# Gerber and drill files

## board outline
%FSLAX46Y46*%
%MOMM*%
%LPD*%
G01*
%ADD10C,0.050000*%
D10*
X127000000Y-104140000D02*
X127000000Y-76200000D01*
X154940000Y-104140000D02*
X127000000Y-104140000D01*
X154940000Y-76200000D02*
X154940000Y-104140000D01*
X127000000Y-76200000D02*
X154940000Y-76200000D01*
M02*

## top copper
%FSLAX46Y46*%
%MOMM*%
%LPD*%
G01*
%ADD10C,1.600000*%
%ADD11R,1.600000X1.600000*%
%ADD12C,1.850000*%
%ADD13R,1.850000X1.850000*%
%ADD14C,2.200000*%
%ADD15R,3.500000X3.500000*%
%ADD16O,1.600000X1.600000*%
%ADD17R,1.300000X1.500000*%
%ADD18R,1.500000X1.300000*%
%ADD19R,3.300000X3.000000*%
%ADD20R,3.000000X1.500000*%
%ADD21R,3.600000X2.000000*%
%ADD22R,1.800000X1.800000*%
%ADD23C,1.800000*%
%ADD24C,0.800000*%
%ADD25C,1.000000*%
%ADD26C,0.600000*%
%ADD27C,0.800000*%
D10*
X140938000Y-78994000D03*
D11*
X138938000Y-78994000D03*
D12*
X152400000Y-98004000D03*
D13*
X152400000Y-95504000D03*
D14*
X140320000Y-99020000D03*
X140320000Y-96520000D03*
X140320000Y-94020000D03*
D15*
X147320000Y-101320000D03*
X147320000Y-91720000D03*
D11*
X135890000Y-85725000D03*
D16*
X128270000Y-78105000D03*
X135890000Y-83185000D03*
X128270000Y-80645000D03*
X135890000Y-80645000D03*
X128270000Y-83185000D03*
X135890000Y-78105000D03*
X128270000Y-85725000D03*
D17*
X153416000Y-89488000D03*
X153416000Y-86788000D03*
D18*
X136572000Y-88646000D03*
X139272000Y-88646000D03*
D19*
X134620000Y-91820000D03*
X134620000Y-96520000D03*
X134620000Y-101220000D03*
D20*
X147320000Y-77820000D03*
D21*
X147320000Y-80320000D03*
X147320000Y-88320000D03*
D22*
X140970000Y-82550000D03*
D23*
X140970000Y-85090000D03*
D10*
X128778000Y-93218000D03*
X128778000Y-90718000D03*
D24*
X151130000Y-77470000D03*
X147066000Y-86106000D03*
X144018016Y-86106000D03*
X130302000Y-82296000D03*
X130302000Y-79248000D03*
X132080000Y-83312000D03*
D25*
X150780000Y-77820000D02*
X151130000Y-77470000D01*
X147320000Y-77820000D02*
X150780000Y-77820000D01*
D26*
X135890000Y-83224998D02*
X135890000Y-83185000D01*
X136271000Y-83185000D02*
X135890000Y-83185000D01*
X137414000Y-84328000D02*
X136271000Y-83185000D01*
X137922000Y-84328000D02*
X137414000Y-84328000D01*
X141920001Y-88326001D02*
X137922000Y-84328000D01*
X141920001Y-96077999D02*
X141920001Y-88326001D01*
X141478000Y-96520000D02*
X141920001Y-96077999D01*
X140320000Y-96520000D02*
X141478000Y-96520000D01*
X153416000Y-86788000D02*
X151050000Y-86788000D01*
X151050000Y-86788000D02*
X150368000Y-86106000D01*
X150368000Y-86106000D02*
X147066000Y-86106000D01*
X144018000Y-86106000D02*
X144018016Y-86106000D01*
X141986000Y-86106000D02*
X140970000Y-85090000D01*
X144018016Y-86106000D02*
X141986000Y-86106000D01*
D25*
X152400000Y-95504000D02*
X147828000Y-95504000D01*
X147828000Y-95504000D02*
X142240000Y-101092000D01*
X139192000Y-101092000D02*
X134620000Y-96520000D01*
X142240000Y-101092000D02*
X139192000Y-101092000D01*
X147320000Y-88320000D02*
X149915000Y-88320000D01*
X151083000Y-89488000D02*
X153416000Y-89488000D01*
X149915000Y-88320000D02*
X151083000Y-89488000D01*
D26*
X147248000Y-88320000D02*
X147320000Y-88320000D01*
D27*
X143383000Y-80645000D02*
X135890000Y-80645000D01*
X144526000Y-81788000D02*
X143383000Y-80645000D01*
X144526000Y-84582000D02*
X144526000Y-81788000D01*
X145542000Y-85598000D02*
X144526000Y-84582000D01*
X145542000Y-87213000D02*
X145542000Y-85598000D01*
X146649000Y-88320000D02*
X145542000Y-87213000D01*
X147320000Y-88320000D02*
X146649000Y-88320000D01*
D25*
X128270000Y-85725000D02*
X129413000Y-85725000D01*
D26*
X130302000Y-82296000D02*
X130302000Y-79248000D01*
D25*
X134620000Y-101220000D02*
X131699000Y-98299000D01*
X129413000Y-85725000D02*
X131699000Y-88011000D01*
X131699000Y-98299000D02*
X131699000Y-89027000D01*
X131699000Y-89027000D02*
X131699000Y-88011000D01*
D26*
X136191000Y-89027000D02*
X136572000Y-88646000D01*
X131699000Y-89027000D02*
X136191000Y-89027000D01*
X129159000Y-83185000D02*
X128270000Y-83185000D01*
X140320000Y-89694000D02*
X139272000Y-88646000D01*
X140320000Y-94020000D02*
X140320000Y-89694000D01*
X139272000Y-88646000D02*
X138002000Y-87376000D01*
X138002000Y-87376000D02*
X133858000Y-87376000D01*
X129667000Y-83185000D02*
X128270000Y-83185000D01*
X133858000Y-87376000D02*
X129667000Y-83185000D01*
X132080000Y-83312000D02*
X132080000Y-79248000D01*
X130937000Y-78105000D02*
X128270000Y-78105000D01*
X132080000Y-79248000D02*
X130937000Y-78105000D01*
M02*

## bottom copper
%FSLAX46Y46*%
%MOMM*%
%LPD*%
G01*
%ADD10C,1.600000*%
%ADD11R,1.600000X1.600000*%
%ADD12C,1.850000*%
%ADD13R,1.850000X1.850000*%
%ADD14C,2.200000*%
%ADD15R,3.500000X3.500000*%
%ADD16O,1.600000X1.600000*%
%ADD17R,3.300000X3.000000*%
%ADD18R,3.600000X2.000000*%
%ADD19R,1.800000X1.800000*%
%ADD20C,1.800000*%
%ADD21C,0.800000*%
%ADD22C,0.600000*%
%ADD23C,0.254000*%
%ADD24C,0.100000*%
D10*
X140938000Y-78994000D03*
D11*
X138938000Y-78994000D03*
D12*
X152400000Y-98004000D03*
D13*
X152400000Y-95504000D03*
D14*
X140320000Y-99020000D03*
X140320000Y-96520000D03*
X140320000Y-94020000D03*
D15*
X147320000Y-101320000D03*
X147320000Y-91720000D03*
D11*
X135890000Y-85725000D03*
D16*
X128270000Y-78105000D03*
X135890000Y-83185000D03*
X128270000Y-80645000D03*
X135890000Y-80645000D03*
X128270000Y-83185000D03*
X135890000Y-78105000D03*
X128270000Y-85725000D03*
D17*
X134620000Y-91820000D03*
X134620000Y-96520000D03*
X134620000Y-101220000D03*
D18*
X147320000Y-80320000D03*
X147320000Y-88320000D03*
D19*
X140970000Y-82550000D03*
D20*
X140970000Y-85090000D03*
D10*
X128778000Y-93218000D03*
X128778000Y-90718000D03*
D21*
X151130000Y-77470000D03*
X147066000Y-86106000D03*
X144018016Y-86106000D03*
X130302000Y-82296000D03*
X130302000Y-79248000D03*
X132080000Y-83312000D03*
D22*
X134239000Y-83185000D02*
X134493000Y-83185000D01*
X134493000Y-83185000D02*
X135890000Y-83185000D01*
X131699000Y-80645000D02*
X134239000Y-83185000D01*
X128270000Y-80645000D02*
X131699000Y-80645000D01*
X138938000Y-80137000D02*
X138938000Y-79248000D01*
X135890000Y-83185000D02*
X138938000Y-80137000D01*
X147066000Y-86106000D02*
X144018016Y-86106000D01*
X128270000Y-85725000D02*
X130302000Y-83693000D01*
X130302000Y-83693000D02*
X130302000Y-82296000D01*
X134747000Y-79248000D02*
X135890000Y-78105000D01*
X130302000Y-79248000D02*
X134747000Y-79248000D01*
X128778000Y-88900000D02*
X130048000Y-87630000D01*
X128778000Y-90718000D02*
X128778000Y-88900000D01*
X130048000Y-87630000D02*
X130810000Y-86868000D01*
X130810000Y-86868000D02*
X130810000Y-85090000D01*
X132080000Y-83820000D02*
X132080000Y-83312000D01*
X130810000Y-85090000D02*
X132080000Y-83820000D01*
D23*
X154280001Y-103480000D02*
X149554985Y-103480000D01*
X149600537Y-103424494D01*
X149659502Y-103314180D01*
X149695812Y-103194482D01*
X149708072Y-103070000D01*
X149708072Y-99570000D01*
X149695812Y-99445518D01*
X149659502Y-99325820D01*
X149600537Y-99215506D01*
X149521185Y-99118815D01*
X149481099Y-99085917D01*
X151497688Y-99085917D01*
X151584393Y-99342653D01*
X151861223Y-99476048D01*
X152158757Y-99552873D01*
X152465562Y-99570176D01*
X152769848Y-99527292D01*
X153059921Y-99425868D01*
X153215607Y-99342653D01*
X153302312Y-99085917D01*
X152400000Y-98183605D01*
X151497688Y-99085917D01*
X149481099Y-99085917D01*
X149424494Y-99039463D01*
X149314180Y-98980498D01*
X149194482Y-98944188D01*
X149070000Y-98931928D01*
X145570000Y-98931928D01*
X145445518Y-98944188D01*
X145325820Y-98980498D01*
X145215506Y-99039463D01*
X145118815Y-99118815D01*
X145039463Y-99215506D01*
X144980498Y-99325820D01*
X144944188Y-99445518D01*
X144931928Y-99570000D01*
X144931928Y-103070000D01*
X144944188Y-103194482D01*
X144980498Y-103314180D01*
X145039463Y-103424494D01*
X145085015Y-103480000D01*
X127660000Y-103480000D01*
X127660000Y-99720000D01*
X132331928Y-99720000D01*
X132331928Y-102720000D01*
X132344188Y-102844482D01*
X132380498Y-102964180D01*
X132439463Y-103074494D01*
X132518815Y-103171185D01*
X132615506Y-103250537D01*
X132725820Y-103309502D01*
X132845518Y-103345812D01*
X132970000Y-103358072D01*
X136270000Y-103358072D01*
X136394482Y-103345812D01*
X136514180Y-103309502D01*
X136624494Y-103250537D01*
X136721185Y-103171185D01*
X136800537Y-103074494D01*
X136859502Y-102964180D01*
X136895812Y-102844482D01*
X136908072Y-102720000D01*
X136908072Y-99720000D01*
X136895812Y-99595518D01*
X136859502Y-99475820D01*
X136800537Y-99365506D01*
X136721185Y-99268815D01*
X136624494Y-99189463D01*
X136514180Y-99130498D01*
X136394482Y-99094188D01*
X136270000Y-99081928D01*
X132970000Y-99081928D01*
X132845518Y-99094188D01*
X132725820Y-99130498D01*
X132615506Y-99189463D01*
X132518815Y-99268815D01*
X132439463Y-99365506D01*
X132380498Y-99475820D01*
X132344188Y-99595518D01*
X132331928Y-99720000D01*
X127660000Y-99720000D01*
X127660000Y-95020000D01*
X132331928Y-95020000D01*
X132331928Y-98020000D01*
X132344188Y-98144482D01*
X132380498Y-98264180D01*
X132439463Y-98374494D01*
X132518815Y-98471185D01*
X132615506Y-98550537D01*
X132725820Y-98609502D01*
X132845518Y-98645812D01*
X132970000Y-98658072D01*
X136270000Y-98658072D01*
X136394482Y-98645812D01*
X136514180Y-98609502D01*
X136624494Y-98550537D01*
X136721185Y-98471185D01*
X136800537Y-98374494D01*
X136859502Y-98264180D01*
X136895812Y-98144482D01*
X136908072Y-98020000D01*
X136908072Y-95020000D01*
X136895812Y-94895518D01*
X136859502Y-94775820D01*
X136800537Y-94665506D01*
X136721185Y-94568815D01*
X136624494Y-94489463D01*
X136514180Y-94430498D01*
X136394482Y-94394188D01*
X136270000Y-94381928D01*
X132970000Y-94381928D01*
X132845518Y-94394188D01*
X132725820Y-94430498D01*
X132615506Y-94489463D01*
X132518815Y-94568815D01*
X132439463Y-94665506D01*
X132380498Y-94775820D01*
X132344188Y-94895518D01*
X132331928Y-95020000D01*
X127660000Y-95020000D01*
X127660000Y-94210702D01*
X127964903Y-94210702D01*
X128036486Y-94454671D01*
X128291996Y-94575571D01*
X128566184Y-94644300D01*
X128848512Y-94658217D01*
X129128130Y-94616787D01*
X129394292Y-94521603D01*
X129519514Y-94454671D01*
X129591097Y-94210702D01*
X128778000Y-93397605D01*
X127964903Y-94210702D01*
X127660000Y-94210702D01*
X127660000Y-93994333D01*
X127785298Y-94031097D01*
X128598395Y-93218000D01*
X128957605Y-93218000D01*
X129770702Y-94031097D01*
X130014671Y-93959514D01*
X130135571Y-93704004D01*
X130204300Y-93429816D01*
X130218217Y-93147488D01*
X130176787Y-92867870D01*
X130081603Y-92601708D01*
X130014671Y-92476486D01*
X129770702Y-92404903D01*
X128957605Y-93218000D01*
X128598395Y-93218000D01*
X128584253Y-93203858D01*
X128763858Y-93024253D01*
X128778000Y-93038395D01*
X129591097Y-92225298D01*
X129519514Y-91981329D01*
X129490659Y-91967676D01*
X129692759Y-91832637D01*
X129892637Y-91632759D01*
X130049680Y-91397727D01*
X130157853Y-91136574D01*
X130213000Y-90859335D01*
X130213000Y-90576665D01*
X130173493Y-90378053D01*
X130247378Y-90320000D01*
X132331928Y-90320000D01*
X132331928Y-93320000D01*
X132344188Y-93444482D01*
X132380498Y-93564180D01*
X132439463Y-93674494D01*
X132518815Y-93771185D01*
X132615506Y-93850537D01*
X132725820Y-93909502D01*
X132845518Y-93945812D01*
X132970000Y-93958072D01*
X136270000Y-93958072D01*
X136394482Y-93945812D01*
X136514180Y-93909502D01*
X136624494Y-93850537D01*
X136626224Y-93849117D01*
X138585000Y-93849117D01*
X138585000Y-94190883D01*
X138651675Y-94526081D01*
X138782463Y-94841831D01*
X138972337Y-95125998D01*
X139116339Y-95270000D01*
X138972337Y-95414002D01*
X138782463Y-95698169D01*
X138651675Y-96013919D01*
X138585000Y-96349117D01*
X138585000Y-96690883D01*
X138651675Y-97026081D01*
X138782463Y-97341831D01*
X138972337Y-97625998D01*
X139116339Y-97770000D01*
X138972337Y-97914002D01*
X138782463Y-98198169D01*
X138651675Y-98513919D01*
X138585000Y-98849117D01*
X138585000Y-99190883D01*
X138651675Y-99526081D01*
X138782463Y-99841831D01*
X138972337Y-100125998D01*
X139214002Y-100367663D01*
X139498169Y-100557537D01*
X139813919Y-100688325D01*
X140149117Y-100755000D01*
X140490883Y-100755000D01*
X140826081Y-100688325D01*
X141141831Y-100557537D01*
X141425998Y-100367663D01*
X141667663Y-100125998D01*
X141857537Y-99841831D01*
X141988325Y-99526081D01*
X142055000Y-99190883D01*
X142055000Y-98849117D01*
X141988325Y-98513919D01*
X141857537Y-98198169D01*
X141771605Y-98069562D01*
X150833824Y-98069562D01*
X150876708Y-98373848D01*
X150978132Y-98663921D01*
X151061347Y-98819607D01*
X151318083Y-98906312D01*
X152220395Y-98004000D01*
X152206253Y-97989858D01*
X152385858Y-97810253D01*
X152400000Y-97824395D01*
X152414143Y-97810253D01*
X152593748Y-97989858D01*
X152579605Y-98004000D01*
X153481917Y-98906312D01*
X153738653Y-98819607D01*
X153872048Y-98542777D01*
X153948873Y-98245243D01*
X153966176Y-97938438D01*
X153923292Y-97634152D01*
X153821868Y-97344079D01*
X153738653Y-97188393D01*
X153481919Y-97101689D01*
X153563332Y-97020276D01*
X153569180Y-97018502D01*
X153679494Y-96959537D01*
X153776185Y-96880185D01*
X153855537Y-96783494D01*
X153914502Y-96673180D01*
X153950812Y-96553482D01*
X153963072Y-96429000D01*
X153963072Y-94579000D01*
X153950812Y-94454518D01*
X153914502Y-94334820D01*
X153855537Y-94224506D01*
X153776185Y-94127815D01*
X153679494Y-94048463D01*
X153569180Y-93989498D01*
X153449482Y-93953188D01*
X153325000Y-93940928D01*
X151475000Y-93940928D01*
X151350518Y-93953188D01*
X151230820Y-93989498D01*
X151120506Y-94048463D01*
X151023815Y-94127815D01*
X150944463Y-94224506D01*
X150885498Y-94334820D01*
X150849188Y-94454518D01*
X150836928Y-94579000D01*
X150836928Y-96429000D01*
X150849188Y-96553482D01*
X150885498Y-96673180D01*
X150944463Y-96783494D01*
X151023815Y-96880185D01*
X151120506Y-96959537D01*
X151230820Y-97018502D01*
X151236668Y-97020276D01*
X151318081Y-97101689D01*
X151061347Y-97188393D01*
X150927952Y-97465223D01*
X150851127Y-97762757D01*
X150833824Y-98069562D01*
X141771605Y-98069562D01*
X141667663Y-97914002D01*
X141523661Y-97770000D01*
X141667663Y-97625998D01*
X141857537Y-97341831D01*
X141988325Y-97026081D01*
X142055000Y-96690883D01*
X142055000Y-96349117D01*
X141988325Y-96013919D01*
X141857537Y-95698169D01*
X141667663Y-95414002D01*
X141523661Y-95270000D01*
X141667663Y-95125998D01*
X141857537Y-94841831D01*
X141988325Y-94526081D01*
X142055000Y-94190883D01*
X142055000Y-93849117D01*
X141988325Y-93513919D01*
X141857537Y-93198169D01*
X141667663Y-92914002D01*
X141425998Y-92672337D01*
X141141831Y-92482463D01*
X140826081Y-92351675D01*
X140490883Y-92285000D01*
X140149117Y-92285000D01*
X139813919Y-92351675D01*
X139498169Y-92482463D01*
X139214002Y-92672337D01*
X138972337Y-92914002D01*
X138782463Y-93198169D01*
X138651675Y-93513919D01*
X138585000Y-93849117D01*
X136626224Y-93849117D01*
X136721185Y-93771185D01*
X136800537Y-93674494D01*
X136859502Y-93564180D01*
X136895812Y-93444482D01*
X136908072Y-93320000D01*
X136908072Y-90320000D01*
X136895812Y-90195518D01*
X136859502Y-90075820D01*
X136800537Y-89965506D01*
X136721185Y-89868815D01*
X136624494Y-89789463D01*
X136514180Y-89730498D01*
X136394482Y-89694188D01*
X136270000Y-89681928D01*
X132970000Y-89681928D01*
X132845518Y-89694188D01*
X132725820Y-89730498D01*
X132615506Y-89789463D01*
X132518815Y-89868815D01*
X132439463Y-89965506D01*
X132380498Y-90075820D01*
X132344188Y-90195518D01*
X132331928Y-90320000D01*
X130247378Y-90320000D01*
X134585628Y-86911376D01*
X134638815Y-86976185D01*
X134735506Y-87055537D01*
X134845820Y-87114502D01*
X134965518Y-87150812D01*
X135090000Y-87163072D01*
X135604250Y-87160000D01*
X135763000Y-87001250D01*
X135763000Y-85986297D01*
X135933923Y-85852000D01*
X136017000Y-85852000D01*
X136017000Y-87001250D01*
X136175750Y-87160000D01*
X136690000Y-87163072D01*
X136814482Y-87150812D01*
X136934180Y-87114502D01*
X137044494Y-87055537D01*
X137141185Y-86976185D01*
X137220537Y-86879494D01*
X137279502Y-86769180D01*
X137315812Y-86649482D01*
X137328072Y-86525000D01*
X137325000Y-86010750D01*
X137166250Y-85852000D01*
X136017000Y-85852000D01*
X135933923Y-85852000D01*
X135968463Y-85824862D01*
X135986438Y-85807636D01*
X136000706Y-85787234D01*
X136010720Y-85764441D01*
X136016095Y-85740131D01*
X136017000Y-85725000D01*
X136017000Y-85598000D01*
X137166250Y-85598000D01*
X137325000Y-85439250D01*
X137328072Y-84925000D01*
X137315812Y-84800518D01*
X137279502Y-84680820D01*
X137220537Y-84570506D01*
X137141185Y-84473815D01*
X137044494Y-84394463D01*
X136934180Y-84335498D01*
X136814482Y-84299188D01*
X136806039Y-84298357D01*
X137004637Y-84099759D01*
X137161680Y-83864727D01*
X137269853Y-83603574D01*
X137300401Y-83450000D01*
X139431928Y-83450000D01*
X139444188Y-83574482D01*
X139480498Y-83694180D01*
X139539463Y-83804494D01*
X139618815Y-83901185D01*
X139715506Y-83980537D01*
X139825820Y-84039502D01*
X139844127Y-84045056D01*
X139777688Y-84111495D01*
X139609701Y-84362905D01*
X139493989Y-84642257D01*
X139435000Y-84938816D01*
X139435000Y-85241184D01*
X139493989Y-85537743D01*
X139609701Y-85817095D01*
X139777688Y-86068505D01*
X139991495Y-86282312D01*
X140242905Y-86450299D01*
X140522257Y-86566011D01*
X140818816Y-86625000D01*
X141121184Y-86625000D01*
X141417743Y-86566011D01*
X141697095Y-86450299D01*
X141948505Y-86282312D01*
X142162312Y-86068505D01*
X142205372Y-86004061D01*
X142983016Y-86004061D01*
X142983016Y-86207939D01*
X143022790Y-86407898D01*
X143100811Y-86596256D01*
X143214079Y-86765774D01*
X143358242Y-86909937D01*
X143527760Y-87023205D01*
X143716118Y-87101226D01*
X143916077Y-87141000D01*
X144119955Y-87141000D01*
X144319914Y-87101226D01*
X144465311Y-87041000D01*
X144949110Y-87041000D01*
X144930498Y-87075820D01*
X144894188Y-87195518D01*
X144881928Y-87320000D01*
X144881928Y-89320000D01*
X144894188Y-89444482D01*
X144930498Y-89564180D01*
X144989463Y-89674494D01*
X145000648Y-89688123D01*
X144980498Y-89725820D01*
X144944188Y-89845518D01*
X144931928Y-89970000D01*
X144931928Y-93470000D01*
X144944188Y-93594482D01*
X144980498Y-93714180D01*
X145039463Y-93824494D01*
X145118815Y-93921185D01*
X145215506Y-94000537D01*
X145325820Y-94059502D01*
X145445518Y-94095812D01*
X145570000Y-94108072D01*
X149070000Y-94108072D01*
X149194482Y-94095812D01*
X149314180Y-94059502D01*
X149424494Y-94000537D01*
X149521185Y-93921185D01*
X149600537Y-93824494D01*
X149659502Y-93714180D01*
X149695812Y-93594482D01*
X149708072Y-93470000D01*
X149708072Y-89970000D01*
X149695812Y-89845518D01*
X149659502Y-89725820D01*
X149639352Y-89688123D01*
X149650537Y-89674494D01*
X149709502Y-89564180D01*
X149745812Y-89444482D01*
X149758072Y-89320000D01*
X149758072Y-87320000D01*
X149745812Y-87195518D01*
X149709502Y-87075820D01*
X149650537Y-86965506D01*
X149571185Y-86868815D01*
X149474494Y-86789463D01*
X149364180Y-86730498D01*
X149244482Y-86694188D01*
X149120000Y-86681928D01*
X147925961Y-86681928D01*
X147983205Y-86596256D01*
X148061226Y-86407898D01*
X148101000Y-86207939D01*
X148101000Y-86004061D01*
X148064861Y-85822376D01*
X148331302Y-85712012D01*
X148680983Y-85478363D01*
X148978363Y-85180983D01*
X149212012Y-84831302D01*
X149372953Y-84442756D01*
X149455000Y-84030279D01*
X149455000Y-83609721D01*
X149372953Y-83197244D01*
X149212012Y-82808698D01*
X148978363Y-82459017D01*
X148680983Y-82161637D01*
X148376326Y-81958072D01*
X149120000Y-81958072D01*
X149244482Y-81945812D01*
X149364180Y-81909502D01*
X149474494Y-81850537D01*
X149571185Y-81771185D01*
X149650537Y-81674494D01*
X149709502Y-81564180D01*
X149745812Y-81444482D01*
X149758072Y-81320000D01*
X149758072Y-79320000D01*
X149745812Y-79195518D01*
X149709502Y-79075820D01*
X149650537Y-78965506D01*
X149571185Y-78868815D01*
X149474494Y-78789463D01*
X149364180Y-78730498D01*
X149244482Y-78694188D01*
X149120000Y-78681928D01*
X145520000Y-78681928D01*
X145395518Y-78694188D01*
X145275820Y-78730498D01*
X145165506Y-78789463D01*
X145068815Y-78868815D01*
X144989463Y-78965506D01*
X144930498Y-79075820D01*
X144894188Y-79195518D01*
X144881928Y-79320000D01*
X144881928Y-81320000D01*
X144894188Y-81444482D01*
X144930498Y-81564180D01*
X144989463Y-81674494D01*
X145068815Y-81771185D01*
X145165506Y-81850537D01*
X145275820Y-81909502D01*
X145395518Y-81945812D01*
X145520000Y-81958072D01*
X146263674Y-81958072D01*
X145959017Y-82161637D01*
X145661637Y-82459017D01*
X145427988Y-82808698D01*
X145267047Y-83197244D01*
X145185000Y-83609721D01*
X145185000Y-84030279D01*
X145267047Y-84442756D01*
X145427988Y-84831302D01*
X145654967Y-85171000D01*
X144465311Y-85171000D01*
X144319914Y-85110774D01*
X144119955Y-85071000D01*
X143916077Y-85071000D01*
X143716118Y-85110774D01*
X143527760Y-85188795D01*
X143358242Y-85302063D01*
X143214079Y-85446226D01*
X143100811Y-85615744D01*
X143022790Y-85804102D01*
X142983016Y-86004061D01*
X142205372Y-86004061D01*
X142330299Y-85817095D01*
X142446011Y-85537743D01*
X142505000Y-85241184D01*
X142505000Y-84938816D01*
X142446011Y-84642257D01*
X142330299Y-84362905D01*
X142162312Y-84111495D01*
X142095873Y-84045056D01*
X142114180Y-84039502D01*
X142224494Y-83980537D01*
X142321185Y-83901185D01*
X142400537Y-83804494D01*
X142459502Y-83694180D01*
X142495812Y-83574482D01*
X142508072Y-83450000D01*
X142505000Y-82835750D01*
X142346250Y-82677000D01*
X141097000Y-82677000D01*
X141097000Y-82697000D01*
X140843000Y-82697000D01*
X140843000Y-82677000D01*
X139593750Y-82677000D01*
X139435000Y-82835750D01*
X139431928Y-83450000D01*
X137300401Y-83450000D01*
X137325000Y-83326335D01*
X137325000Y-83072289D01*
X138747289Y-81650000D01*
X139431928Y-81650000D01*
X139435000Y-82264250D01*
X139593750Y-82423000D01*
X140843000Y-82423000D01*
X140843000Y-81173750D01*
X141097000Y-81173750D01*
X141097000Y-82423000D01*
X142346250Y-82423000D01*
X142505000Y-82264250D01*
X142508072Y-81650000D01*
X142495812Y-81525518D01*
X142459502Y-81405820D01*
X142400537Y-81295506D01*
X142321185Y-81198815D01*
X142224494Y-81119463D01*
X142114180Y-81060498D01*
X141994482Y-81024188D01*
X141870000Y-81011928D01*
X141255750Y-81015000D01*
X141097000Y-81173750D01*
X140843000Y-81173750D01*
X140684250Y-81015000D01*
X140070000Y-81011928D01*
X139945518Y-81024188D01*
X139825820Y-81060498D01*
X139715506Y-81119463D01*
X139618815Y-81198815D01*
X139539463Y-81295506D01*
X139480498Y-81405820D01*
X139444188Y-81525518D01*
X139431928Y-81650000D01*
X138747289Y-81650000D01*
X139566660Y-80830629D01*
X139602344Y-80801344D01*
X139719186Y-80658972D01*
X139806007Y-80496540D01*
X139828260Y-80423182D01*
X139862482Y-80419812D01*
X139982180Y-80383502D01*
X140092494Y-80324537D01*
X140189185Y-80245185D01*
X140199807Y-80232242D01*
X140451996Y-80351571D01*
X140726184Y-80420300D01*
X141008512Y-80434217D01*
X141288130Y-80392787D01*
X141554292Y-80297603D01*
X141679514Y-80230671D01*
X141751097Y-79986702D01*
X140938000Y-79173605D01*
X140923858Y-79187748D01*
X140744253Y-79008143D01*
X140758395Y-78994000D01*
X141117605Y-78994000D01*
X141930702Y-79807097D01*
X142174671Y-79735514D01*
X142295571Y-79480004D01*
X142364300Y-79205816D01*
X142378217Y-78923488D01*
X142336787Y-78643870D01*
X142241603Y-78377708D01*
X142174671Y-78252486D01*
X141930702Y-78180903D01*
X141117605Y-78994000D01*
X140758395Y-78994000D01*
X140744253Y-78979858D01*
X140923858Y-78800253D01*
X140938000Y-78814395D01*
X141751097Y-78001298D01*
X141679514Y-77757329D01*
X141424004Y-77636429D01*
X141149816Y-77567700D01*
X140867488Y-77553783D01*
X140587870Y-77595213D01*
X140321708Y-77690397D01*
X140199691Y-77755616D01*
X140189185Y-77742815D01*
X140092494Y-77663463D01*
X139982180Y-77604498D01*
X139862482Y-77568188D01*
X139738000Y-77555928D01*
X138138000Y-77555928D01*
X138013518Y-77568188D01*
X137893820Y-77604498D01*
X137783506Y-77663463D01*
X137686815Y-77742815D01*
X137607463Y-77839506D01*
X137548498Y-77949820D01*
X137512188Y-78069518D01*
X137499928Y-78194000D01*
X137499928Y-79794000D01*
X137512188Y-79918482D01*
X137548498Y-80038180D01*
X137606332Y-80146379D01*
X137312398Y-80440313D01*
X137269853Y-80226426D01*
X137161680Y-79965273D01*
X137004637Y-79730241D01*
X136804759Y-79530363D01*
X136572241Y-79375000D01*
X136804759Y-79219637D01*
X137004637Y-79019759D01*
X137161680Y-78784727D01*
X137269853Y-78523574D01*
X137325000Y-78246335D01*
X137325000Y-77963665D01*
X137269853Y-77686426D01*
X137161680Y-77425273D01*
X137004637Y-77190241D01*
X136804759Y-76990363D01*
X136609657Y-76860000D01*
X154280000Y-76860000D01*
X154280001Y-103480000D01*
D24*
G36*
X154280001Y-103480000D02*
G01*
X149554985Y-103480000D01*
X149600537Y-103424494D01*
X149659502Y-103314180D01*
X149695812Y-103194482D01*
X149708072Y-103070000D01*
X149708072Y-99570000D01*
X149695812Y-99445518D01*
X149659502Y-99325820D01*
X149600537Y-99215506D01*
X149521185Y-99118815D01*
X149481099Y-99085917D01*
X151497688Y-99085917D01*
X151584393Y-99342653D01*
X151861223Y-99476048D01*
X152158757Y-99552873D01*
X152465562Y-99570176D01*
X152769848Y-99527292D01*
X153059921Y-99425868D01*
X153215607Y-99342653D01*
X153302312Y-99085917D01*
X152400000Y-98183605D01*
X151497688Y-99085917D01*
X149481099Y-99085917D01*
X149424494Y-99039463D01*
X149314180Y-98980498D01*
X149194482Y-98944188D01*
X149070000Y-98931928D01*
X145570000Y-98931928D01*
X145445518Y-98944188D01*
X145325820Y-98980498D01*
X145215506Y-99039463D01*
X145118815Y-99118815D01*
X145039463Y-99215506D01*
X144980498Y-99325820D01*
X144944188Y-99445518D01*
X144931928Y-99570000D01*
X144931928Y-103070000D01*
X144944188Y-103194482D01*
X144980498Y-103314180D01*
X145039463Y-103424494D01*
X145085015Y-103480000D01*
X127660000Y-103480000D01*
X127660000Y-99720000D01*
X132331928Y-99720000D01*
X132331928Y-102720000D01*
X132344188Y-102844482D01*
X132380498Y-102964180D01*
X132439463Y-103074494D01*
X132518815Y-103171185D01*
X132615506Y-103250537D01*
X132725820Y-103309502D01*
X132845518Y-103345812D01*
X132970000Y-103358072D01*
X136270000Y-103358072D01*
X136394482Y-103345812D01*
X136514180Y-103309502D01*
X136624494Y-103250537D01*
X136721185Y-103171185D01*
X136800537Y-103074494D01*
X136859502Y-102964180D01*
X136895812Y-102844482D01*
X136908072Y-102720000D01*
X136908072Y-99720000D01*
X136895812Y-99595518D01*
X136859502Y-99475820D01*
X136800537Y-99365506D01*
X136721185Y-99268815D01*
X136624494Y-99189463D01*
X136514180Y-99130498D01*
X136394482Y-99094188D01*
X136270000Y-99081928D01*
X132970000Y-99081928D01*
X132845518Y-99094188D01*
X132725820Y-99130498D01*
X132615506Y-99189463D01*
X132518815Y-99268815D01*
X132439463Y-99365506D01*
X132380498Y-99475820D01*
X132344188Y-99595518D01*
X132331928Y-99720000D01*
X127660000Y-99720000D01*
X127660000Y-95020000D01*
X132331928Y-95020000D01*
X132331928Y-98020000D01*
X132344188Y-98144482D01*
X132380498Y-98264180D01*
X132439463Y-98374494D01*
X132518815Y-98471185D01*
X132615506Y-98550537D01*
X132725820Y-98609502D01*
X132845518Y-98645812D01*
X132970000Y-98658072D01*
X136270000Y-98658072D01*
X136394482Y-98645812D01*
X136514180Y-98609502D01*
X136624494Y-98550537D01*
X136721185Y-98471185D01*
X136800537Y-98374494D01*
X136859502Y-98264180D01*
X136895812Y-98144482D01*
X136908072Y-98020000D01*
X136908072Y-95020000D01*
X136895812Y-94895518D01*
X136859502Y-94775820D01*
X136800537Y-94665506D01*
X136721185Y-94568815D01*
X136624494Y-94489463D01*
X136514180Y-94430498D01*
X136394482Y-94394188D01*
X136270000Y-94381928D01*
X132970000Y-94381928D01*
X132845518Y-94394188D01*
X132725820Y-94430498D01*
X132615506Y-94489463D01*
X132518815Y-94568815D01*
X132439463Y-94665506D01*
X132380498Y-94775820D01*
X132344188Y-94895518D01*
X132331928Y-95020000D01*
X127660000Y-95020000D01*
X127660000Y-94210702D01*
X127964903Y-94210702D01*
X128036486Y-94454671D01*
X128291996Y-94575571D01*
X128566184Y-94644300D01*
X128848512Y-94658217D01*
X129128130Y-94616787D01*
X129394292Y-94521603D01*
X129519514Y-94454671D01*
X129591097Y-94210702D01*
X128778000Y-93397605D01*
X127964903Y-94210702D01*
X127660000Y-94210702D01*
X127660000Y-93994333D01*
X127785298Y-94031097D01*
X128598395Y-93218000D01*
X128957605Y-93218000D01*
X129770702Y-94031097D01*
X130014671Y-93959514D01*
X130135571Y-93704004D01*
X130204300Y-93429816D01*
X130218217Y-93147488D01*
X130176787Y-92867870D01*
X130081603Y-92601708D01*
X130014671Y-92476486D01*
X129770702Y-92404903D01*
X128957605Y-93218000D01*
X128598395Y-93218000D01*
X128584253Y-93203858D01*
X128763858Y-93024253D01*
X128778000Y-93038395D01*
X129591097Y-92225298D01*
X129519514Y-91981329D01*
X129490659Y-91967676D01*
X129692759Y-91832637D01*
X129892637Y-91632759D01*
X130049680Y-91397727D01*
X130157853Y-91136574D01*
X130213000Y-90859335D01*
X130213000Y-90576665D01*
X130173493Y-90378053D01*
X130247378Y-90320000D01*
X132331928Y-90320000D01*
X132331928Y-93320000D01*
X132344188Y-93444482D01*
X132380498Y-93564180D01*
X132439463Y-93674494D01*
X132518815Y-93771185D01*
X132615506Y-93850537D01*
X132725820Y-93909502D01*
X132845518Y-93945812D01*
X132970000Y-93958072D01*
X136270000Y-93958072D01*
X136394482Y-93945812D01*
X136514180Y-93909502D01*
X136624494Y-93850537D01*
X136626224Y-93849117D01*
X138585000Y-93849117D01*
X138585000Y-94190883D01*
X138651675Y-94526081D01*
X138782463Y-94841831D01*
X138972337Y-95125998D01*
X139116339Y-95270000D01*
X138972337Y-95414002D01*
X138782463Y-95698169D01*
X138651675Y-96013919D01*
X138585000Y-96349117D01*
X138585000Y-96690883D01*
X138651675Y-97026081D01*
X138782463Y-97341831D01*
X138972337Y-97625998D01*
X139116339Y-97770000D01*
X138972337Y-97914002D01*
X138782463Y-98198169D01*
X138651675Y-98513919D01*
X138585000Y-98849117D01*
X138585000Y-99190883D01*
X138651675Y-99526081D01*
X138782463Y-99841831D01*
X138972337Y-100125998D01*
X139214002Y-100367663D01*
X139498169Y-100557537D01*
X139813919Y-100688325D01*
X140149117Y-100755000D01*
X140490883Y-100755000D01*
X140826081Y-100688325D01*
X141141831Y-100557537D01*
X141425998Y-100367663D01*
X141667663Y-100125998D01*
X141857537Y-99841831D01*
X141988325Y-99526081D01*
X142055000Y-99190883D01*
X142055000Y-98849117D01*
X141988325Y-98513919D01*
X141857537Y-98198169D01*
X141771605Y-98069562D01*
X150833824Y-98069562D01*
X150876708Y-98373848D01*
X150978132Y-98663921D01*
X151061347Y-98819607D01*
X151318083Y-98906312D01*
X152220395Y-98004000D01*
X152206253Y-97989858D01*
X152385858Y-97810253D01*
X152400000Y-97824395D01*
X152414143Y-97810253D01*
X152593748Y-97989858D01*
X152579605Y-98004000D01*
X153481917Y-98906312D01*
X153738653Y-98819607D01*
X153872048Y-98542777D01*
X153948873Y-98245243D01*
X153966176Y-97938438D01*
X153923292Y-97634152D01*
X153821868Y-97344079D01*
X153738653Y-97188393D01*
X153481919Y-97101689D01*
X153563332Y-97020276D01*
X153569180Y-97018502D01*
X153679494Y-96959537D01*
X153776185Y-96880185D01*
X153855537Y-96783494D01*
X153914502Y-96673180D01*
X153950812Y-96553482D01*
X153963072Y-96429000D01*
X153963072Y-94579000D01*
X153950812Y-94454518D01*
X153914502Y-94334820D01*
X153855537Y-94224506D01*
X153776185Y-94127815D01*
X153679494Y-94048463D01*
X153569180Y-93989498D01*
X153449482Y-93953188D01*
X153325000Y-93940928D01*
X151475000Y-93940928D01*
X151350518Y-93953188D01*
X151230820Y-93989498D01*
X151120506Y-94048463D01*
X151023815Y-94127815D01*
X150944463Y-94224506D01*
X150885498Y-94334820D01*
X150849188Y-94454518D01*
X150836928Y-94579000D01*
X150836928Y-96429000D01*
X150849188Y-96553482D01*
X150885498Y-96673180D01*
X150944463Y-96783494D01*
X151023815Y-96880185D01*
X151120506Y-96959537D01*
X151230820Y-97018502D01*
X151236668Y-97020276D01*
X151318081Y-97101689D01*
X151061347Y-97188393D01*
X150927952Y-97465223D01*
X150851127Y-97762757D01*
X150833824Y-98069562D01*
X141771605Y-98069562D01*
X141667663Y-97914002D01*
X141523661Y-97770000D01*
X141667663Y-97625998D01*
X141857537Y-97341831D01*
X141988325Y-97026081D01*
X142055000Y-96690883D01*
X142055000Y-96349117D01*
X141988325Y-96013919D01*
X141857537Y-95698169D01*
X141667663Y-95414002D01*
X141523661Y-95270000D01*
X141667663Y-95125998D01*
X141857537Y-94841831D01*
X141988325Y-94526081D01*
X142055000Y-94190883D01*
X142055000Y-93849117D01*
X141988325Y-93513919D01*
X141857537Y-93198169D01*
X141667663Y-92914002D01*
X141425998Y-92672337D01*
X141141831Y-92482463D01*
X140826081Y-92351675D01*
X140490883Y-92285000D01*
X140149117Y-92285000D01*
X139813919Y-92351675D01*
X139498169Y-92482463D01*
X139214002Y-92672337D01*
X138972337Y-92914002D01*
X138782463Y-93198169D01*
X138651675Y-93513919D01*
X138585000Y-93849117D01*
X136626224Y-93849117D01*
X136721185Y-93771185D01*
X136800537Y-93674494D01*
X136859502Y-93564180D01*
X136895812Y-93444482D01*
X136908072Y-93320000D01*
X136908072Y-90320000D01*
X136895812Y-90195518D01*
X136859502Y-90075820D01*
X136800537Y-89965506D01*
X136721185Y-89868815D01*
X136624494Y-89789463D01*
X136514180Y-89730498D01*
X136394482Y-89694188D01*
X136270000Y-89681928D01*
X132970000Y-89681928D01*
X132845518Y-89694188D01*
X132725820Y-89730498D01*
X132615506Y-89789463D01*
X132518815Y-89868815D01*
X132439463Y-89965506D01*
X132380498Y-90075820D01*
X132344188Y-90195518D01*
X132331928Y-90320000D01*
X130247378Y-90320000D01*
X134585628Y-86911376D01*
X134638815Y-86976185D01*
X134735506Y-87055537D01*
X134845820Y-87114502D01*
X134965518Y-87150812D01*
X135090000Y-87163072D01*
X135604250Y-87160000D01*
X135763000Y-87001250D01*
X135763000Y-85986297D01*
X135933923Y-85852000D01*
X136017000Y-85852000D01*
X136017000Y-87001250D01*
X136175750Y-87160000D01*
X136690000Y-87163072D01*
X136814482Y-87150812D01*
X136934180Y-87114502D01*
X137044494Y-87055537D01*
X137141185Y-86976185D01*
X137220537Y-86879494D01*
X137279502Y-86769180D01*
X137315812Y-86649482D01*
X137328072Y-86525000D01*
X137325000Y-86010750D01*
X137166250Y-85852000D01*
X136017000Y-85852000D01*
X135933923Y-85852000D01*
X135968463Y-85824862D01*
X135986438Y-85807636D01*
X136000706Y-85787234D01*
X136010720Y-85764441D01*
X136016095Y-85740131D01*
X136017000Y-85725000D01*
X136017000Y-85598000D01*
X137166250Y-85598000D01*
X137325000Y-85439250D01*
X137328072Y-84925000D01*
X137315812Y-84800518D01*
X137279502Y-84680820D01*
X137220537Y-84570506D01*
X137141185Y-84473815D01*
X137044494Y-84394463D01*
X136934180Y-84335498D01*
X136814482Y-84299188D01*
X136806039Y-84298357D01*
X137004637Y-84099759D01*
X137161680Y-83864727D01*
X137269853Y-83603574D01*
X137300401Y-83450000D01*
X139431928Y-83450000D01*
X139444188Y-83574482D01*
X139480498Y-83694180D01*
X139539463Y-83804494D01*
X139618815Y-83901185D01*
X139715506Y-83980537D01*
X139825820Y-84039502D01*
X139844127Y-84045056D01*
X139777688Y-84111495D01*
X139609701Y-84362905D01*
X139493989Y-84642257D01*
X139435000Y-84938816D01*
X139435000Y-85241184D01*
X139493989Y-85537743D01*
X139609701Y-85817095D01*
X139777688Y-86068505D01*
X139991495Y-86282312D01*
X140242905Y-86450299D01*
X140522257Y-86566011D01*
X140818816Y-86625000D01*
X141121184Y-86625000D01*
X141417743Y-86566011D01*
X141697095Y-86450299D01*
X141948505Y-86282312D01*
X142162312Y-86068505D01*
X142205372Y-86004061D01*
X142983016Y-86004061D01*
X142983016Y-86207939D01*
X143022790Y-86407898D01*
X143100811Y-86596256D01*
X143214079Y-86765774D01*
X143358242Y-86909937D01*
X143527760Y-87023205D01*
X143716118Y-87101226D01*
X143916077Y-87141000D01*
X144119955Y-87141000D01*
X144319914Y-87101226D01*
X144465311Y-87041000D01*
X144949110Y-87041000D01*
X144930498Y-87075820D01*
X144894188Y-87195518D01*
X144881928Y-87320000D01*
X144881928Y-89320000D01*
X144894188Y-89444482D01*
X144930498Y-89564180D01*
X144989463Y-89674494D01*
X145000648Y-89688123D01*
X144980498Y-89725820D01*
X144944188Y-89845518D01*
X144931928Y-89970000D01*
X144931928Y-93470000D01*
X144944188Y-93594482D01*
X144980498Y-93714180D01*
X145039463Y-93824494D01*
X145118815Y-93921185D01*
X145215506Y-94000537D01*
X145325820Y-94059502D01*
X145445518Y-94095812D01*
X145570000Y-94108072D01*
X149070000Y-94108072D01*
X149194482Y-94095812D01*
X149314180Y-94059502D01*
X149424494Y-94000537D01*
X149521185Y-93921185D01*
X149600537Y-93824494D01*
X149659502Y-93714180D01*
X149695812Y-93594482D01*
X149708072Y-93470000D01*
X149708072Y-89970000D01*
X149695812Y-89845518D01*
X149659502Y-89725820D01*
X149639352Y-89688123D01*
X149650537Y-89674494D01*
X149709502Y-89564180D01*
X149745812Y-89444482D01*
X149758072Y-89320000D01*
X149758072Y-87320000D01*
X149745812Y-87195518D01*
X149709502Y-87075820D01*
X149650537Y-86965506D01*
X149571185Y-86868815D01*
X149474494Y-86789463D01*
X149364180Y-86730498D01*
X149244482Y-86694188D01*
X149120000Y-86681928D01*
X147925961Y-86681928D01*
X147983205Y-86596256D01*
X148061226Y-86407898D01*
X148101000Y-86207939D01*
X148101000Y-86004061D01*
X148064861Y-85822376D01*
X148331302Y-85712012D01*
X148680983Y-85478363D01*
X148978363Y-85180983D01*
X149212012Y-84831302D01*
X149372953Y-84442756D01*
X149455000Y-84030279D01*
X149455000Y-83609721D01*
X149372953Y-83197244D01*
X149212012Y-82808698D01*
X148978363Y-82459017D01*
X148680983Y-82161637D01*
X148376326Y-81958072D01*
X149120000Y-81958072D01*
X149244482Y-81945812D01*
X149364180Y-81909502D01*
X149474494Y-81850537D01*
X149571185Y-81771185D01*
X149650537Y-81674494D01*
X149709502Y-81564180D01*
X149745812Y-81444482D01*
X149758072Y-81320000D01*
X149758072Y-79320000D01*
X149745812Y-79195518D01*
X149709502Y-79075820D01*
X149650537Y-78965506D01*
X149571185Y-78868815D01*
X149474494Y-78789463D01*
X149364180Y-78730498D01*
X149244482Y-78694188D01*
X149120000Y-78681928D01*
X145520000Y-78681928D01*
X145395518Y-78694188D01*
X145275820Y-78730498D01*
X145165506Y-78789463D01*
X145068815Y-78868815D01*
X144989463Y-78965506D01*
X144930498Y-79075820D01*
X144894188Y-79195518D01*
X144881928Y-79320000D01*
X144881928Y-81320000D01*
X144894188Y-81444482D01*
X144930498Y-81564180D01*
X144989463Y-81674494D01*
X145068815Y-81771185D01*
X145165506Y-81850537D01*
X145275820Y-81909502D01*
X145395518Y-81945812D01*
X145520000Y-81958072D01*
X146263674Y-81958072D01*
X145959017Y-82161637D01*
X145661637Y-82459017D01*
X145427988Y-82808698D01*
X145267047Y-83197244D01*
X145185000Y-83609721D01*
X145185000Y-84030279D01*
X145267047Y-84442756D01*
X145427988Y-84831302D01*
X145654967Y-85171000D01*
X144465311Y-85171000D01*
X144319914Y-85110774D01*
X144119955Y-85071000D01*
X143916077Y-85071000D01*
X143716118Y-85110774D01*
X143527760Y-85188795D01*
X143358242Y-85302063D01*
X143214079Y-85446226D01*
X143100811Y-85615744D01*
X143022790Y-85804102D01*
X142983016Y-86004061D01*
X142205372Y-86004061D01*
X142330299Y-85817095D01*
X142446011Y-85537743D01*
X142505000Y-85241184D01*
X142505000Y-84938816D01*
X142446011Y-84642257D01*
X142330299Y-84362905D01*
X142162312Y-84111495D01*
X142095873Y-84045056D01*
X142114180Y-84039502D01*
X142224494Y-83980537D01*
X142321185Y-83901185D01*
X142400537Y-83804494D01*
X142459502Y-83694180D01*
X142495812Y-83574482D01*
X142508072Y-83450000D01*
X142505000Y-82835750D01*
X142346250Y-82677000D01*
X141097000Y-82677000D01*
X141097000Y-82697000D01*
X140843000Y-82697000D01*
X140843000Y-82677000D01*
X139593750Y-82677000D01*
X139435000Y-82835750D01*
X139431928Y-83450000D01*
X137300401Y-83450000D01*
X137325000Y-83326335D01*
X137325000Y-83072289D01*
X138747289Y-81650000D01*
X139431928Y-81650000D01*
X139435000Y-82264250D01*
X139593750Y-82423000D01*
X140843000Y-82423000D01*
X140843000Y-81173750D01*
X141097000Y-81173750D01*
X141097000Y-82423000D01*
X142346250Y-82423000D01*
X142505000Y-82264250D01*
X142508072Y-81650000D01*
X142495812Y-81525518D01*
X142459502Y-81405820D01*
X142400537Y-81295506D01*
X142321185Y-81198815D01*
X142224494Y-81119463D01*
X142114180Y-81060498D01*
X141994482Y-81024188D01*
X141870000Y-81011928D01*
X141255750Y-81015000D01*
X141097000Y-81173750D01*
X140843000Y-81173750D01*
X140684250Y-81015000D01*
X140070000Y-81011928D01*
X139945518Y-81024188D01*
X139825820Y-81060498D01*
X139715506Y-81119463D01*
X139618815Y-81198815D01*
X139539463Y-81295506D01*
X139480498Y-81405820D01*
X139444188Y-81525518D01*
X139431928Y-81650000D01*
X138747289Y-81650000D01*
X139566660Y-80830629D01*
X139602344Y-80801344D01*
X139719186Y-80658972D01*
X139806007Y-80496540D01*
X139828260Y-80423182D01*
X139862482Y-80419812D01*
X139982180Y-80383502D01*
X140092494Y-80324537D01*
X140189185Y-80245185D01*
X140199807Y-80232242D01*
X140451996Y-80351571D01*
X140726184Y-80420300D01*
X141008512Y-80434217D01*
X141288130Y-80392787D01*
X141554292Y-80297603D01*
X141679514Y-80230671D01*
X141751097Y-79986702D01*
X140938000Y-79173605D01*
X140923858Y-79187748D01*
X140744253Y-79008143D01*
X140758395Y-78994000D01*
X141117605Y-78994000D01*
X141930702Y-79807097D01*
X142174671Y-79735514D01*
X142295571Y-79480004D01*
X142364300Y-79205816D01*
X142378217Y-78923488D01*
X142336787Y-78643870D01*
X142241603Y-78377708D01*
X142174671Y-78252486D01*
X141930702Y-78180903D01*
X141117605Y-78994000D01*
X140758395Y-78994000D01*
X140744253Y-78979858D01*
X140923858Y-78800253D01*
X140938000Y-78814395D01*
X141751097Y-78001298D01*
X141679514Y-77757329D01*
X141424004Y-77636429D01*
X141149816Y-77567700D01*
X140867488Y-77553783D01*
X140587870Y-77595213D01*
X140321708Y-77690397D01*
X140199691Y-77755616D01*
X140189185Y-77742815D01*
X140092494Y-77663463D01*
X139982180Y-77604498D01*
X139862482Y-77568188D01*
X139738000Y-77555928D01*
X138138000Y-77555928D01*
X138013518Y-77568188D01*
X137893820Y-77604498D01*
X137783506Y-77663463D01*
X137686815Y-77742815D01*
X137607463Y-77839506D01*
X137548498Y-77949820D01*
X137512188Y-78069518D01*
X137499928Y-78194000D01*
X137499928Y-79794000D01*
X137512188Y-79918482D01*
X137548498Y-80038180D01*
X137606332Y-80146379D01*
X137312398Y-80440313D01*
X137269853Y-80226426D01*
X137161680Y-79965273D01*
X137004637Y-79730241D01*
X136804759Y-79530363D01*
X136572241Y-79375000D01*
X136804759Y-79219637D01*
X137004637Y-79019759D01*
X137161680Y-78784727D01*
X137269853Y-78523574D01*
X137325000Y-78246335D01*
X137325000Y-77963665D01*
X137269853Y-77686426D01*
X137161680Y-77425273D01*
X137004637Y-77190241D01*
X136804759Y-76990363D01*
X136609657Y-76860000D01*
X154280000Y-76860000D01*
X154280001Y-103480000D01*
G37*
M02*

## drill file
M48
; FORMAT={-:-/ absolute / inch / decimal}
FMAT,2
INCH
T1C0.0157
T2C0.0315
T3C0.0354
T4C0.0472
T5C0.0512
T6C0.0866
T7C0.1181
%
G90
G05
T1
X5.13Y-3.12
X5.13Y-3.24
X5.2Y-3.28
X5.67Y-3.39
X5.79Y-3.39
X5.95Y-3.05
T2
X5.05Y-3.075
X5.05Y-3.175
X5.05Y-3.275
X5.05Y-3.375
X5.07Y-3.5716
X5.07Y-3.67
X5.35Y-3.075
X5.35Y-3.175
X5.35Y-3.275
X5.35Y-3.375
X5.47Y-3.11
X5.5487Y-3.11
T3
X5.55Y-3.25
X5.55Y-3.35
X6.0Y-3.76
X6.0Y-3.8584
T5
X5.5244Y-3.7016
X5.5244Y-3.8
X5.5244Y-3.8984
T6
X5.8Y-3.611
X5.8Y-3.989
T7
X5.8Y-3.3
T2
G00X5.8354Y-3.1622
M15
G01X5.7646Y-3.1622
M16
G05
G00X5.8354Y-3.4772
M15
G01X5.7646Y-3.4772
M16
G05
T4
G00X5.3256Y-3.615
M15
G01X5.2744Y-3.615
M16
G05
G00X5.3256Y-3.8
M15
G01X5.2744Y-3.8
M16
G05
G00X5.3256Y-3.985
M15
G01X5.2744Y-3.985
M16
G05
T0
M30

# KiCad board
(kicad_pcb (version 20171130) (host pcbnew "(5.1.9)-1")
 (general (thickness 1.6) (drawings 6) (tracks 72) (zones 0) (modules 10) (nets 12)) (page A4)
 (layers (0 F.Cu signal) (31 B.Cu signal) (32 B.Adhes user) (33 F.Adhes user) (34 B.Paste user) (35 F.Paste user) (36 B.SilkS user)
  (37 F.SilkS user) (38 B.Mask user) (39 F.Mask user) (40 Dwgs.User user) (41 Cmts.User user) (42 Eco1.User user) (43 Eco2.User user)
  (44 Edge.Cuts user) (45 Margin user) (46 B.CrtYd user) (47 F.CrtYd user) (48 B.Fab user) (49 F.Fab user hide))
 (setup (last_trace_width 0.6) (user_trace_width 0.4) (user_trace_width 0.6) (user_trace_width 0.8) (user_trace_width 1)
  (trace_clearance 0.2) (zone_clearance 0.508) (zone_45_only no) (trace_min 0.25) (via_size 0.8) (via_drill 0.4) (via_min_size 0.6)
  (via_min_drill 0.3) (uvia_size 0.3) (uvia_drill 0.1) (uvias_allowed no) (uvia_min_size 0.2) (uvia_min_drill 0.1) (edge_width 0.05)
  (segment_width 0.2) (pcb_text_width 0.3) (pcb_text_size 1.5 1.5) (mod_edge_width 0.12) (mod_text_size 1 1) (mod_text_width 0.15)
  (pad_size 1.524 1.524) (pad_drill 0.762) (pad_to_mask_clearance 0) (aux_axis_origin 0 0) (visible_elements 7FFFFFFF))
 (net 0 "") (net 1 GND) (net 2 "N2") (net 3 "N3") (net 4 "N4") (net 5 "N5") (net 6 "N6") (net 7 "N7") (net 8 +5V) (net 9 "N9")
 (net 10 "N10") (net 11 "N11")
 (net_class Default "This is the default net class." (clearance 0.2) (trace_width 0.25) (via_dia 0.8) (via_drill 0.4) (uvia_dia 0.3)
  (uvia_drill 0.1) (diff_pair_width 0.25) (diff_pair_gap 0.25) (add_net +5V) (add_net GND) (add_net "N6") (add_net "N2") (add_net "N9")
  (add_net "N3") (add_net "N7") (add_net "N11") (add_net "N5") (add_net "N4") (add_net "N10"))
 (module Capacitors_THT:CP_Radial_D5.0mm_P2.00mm (layer F.Cu) (at 138.938 78.994)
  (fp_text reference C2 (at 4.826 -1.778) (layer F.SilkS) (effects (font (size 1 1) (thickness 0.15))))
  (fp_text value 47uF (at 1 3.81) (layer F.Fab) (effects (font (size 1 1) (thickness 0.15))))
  (pad 2 thru_hole circle (at 2 0) (size 1.6 1.6) (drill 0.8) (layers *.Cu *.Mask) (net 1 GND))
  (pad 1 thru_hole rect (at 0 0) (size 1.6 1.6) (drill 0.8) (layers *.Cu *.Mask) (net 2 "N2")))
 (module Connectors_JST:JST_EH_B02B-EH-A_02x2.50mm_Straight (layer F.Cu) (at 152.4 95.504 270)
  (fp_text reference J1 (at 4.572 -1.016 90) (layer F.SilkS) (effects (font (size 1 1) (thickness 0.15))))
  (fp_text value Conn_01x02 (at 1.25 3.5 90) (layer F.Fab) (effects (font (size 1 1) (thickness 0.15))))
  (pad 2 thru_hole circle (at 2.5 0 270) (size 1.85 1.85) (drill 0.9) (layers *.Cu *.Mask) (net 1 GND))
  (pad 1 thru_hole rect (at 0 0 270) (size 1.85 1.85) (drill 0.9) (layers *.Cu *.Mask) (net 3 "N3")))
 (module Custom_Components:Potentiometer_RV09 (layer F.Cu) (at 147.32 96.52 270)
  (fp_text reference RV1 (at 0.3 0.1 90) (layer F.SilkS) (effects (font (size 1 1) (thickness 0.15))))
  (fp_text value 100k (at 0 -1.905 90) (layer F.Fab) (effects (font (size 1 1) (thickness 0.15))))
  (pad 3 thru_hole circle (at 2.5 7 270) (size 2.2 2.2) (drill 1.3) (layers *.Cu *.Mask) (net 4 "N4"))
  (pad 2 thru_hole circle (at 0 7 270) (size 2.2 2.2) (drill 1.3) (layers *.Cu *.Mask) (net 2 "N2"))
  (pad 1 thru_hole circle (at -2.5 7 270) (size 2.2 2.2) (drill 1.3) (layers *.Cu *.Mask) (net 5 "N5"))
  (pad 0 thru_hole rect (at 4.8 0 270) (size 3.5 3.5) (drill 2.2) (layers *.Cu *.Mask))
  (pad 0 thru_hole rect (at -4.8 0 270) (size 3.5 3.5) (drill 2.2) (layers *.Cu *.Mask)))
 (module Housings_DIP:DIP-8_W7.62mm (layer F.Cu) (at 135.89 85.725 180)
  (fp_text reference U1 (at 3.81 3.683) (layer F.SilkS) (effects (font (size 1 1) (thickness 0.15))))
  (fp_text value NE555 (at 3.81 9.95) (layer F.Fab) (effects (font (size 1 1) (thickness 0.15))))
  (pad 1 thru_hole rect (at 0 0 180) (size 1.6 1.6) (drill 0.8) (layers *.Cu *.Mask) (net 1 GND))
  (pad 5 thru_hole oval (at 7.62 7.62 180) (size 1.6 1.6) (drill 0.8) (layers *.Cu *.Mask) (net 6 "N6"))
  (pad 2 thru_hole oval (at 0 2.54 180) (size 1.6 1.6) (drill 0.8) (layers *.Cu *.Mask) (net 2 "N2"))
  (pad 6 thru_hole oval (at 7.62 5.08 180) (size 1.6 1.6) (drill 0.8) (layers *.Cu *.Mask) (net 2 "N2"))
  (pad 3 thru_hole oval (at 0 5.08 180) (size 1.6 1.6) (drill 0.8) (layers *.Cu *.Mask) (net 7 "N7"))
  (pad 7 thru_hole oval (at 7.62 2.54 180) (size 1.6 1.6) (drill 0.8) (layers *.Cu *.Mask) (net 5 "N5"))
  (pad 4 thru_hole oval (at 0 7.62 180) (size 1.6 1.6) (drill 0.8) (layers *.Cu *.Mask) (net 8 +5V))
  (pad 8 thru_hole oval (at 7.62 0 180) (size 1.6 1.6) (drill 0.8) (layers *.Cu *.Mask) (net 8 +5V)))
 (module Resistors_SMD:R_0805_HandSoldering (layer F.Cu) (at 153.416 88.138 90)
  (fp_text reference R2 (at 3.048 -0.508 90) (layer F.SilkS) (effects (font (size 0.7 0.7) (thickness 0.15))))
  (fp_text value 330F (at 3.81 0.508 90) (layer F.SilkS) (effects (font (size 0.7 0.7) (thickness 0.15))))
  (pad 1 smd rect (at -1.35 0 90) (size 1.5 1.3) (layers F.Cu F.Paste F.Mask) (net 7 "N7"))
  (pad 2 smd rect (at 1.35 0 90) (size 1.5 1.3) (layers F.Cu F.Paste F.Mask) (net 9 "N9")))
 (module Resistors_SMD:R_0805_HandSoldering (layer F.Cu) (at 137.922 88.646)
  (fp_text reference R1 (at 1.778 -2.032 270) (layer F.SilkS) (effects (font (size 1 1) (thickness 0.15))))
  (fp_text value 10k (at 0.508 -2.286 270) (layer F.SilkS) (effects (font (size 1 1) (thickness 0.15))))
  (pad 1 smd rect (at -1.35 0) (size 1.5 1.3) (layers F.Cu F.Paste F.Mask) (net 8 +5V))
  (pad 2 smd rect (at 1.35 0) (size 1.5 1.3) (layers F.Cu F.Paste F.Mask) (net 5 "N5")))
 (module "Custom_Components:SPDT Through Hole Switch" (layer F.Cu) (at 134.62 101.22 180)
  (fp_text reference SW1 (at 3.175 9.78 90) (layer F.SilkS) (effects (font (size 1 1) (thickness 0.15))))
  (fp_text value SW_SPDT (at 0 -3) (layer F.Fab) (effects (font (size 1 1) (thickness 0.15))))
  (pad 3 thru_hole rect (at 0 9.4 180) (size 3.3 3) (drill oval 2.5 1.2) (layers *.Cu *.Mask) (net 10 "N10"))
  (pad 2 thru_hole rect (at 0 4.7 180) (size 3.3 3) (drill oval 2.5 1.2) (layers *.Cu *.Mask) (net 3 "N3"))
  (pad 1 thru_hole rect (at 0 0 180) (size 3.3 3) (drill oval 2.5 1.2) (layers *.Cu *.Mask) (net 8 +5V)))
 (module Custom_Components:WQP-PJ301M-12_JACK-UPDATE (layer F.Cu) (at 147.32 83.82 180)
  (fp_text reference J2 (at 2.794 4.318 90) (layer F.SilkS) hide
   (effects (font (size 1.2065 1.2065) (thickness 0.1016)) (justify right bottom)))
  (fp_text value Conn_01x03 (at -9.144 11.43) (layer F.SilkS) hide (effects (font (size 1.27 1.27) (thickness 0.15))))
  (pad "" np_thru_hole circle (at 0 0 180) (size 3 3) (drill 3) (layers *.Cu *.Mask) (solder_mask_margin 0.1016))
  (pad 3 smd rect (at 0 6 180) (size 3 1.5) (layers F.Cu F.Paste F.Mask) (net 1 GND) (solder_mask_margin 0.1016))
  (pad 2 thru_hole rect (at 0 3.5 180) (size 3.6 2) (drill oval 2.6 0.8) (layers *.Cu *.Mask) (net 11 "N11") (solder_mask_margin 0.1016))
  (pad 1 thru_hole rect (at 0 -4.5 180) (size 3.6 2) (drill oval 2.6 0.8) (layers *.Cu *.Mask) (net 7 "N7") (solder_mask_margin 0.1016)
   (zone_connect 2)))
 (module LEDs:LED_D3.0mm (layer F.Cu) (at 140.97 82.55 270)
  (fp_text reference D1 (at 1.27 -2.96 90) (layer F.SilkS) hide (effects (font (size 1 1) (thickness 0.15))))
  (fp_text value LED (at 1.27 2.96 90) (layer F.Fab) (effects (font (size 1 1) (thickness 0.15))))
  (pad 1 thru_hole rect (at 0 0 270) (size 1.8 1.8) (drill 0.9) (layers *.Cu *.Mask) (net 1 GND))
  (pad 2 thru_hole circle (at 2.54 0 270) (size 1.8 1.8) (drill 0.9) (layers *.Cu *.Mask) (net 9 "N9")))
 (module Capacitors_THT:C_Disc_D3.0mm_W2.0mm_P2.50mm (layer F.Cu) (at 128.778 93.218 90)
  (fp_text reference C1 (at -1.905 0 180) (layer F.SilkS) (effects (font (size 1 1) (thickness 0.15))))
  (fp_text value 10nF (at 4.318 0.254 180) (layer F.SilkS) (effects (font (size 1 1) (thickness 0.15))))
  (pad 1 thru_hole circle (at 0 0 90) (size 1.6 1.6) (drill 0.8) (layers *.Cu *.Mask) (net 1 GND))
  (pad 2 thru_hole circle (at 2.5 0 90) (size 1.6 1.6) (drill 0.8) (layers *.Cu *.Mask) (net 6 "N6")))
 (gr_line (start 127 104.14) (end 127 76.2) (layer Edge.Cuts) (width 0.05))
 (gr_line (start 154.94 104.14) (end 127 104.14) (layer Edge.Cuts) (width 0.05))
 (gr_line (start 154.94 76.2) (end 154.94 104.14) (layer Edge.Cuts) (width 0.05))
 (gr_line (start 127 76.2) (end 154.94 76.2) (layer Edge.Cuts) (width 0.05))
 (via (at 151.13 77.47) (size 0.8) (drill 0.4) (layers F.Cu B.Cu) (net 1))
 (segment (start 150.78 77.82) (end 151.13 77.47) (width 1) (layer F.Cu) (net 1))
 (segment (start 147.32 77.82) (end 150.78 77.82) (width 1) (layer F.Cu) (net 1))
 (segment (start 134.239 83.185) (end 134.493 83.185) (width 0.6) (layer B.Cu) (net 2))
 (segment (start 134.493 83.185) (end 135.89 83.185) (width 0.6) (layer B.Cu) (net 2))
 (segment (start 131.699 80.645) (end 134.239 83.185) (width 0.6) (layer B.Cu) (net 2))
 (segment (start 128.27 80.645) (end 131.699 80.645) (width 0.6) (layer B.Cu) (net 2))
 (segment (start 138.938 80.137) (end 138.938 79.248) (width 0.6) (layer B.Cu) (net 2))
 (segment (start 135.89 83.185) (end 138.938 80.137) (width 0.6) (layer B.Cu) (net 2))
 (segment (start 135.89 83.224998) (end 135.89 83.185) (width 0.6) (layer F.Cu) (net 2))
 (segment (start 136.271 83.185) (end 135.89 83.185) (width 0.6) (layer F.Cu) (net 2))
 (segment (start 137.414 84.328) (end 136.271 83.185) (width 0.6) (layer F.Cu) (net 2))
 (segment (start 137.922 84.328) (end 137.414 84.328) (width 0.6) (layer F.Cu) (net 2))
 (segment (start 141.920001 88.326001) (end 137.922 84.328) (width 0.6) (layer F.Cu) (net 2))
 (segment (start 141.920001 96.077999) (end 141.920001 88.326001) (width 0.6) (layer F.Cu) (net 2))
 (segment (start 141.478 96.52) (end 141.920001 96.077999) (width 0.6) (layer F.Cu) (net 2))
 (segment (start 140.32 96.52) (end 141.478 96.52) (width 0.6) (layer F.Cu) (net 2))
 (segment (start 153.416 86.788) (end 151.05 86.788) (width 0.6) (layer F.Cu) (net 9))
 (segment (start 151.05 86.788) (end 150.368 86.106) (width 0.6) (layer F.Cu) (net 9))
 (via (at 147.066 86.106) (size 0.8) (drill 0.4) (layers F.Cu B.Cu) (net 9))
 (segment (start 150.368 86.106) (end 147.066 86.106) (width 0.6) (layer F.Cu) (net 9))
 (via (at 144.018016 86.106) (size 0.8) (drill 0.4) (layers F.Cu B.Cu) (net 9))
 (segment (start 144.018 86.106) (end 144.018016 86.106) (width 0.6) (layer F.Cu) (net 9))
 (segment (start 147.066 86.106) (end 144.018016 86.106) (width 0.6) (layer B.Cu) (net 9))
 (segment (start 141.986 86.106) (end 140.97 85.09) (width 0.6) (layer F.Cu) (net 9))
 (segment (start 144.018016 86.106) (end 141.986 86.106) (width 0.6) (layer F.Cu) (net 9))
 (segment (start 152.4 95.504) (end 147.828 95.504) (width 1) (layer F.Cu) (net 3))
 (segment (start 147.828 95.504) (end 142.24 101.092) (width 1) (layer F.Cu) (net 3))
 (segment (start 139.192 101.092) (end 134.62 96.52) (width 1) (layer F.Cu) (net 3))
 (segment (start 142.24 101.092) (end 139.192 101.092) (width 1) (layer F.Cu) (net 3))
 (segment (start 147.32 88.32) (end 149.915 88.32) (width 1) (layer F.Cu) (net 7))
 (segment (start 151.083 89.488) (end 153.416 89.488) (width 1) (layer F.Cu) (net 7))
 (segment (start 149.915 88.32) (end 151.083 89.488) (width 1) (layer F.Cu) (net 7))
 (segment (start 147.248 88.32) (end 147.32 88.32) (width 0.6) (layer F.Cu) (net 7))
 (segment (start 143.383 80.645) (end 135.89 80.645) (width 0.8) (layer F.Cu) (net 7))
 (segment (start 144.526 81.788) (end 143.383 80.645) (width 0.8) (layer F.Cu) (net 7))
 (segment (start 144.526 84.582) (end 144.526 81.788) (width 0.8) (layer F.Cu) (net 7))
 (segment (start 145.542 85.598) (end 144.526 84.582) (width 0.8) (layer F.Cu) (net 7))
 (segment (start 145.542 87.213) (end 145.542 85.598) (width 0.8) (layer F.Cu) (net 7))
 (segment (start 146.649 88.32) (end 145.542 87.213) (width 0.8) (layer F.Cu) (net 7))
 (segment (start 147.32 88.32) (end 146.649 88.32) (width 0.8) (layer F.Cu) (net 7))
 (segment (start 128.27 85.725) (end 129.413 85.725) (width 1) (layer F.Cu) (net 8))
 (segment (start 128.27 85.725) (end 130.302 83.693) (width 0.6) (layer B.Cu) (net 8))
 (via (at 130.302 82.296) (size 0.8) (drill 0.4) (layers F.Cu B.Cu) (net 8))
 (segment (start 130.302 83.693) (end 130.302 82.296) (width 0.6) (layer B.Cu) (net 8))
 (via (at 130.302 79.248) (size 0.8) (drill 0.4) (layers F.Cu B.Cu) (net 8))
 (segment (start 130.302 82.296) (end 130.302 79.248) (width 0.6) (layer F.Cu) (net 8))
 (segment (start 134.747 79.248) (end 135.89 78.105) (width 0.6) (layer B.Cu) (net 8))
 (segment (start 130.302 79.248) (end 134.747 79.248) (width 0.6) (layer B.Cu) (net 8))
 (segment (start 134.62 101.22) (end 131.699 98.299) (width 1) (layer F.Cu) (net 8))
 (segment (start 129.413 85.725) (end 131.699 88.011) (width 1) (layer F.Cu) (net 8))
 (segment (start 131.699 98.299) (end 131.699 89.027) (width 1) (layer F.Cu) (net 8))
 (segment (start 131.699 89.027) (end 131.699 88.011) (width 1) (layer F.Cu) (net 8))
 (segment (start 136.191 89.027) (end 136.572 88.646) (width 0.6) (layer F.Cu) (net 8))
 (segment (start 131.699 89.027) (end 136.191 89.027) (width 0.6) (layer F.Cu) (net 8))
 (segment (start 129.159 83.185) (end 128.27 83.185) (width 0.6) (layer F.Cu) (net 5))
 (segment (start 140.32 89.694) (end 139.272 88.646) (width 0.6) (layer F.Cu) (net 5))
 (segment (start 140.32 94.02) (end 140.32 89.694) (width 0.6) (layer F.Cu) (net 5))
 (segment (start 139.272 88.646) (end 138.002 87.376) (width 0.6) (layer F.Cu) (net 5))
 (segment (start 138.002 87.376) (end 133.858 87.376) (width 0.6) (layer F.Cu) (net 5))
 (segment (start 129.667 83.185) (end 128.27 83.185) (width 0.6) (layer F.Cu) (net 5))
 (segment (start 133.858 87.376) (end 129.667 83.185) (width 0.6) (layer F.Cu) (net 5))
 (segment (start 128.778 88.9) (end 130.048 87.63) (width 0.6) (layer B.Cu) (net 6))
 (segment (start 128.778 90.718) (end 128.778 88.9) (width 0.6) (layer B.Cu) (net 6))
 (segment (start 130.048 87.63) (end 130.81 86.868) (width 0.6) (layer B.Cu) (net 6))
 (segment (start 130.81 86.868) (end 130.81 85.09) (width 0.6) (layer B.Cu) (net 6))
 (via (at 132.08 83.312) (size 0.8) (drill 0.4) (layers F.Cu B.Cu) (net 6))
 (segment (start 132.08 83.82) (end 132.08 83.312) (width 0.6) (layer B.Cu) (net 6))
 (segment (start 130.81 85.09) (end 132.08 83.82) (width 0.6) (layer B.Cu) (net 6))
 (segment (start 132.08 83.312) (end 132.08 79.248) (width 0.6) (layer F.Cu) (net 6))
 (segment (start 130.937 78.105) (end 128.27 78.105) (width 0.6) (layer F.Cu) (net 6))
 (segment (start 132.08 79.248) (end 130.937 78.105) (width 0.6) (layer F.Cu) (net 6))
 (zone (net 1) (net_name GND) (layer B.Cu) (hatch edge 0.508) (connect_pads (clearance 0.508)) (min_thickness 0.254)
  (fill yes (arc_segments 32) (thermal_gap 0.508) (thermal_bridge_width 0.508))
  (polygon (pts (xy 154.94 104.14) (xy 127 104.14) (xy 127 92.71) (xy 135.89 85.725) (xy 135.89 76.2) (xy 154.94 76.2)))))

